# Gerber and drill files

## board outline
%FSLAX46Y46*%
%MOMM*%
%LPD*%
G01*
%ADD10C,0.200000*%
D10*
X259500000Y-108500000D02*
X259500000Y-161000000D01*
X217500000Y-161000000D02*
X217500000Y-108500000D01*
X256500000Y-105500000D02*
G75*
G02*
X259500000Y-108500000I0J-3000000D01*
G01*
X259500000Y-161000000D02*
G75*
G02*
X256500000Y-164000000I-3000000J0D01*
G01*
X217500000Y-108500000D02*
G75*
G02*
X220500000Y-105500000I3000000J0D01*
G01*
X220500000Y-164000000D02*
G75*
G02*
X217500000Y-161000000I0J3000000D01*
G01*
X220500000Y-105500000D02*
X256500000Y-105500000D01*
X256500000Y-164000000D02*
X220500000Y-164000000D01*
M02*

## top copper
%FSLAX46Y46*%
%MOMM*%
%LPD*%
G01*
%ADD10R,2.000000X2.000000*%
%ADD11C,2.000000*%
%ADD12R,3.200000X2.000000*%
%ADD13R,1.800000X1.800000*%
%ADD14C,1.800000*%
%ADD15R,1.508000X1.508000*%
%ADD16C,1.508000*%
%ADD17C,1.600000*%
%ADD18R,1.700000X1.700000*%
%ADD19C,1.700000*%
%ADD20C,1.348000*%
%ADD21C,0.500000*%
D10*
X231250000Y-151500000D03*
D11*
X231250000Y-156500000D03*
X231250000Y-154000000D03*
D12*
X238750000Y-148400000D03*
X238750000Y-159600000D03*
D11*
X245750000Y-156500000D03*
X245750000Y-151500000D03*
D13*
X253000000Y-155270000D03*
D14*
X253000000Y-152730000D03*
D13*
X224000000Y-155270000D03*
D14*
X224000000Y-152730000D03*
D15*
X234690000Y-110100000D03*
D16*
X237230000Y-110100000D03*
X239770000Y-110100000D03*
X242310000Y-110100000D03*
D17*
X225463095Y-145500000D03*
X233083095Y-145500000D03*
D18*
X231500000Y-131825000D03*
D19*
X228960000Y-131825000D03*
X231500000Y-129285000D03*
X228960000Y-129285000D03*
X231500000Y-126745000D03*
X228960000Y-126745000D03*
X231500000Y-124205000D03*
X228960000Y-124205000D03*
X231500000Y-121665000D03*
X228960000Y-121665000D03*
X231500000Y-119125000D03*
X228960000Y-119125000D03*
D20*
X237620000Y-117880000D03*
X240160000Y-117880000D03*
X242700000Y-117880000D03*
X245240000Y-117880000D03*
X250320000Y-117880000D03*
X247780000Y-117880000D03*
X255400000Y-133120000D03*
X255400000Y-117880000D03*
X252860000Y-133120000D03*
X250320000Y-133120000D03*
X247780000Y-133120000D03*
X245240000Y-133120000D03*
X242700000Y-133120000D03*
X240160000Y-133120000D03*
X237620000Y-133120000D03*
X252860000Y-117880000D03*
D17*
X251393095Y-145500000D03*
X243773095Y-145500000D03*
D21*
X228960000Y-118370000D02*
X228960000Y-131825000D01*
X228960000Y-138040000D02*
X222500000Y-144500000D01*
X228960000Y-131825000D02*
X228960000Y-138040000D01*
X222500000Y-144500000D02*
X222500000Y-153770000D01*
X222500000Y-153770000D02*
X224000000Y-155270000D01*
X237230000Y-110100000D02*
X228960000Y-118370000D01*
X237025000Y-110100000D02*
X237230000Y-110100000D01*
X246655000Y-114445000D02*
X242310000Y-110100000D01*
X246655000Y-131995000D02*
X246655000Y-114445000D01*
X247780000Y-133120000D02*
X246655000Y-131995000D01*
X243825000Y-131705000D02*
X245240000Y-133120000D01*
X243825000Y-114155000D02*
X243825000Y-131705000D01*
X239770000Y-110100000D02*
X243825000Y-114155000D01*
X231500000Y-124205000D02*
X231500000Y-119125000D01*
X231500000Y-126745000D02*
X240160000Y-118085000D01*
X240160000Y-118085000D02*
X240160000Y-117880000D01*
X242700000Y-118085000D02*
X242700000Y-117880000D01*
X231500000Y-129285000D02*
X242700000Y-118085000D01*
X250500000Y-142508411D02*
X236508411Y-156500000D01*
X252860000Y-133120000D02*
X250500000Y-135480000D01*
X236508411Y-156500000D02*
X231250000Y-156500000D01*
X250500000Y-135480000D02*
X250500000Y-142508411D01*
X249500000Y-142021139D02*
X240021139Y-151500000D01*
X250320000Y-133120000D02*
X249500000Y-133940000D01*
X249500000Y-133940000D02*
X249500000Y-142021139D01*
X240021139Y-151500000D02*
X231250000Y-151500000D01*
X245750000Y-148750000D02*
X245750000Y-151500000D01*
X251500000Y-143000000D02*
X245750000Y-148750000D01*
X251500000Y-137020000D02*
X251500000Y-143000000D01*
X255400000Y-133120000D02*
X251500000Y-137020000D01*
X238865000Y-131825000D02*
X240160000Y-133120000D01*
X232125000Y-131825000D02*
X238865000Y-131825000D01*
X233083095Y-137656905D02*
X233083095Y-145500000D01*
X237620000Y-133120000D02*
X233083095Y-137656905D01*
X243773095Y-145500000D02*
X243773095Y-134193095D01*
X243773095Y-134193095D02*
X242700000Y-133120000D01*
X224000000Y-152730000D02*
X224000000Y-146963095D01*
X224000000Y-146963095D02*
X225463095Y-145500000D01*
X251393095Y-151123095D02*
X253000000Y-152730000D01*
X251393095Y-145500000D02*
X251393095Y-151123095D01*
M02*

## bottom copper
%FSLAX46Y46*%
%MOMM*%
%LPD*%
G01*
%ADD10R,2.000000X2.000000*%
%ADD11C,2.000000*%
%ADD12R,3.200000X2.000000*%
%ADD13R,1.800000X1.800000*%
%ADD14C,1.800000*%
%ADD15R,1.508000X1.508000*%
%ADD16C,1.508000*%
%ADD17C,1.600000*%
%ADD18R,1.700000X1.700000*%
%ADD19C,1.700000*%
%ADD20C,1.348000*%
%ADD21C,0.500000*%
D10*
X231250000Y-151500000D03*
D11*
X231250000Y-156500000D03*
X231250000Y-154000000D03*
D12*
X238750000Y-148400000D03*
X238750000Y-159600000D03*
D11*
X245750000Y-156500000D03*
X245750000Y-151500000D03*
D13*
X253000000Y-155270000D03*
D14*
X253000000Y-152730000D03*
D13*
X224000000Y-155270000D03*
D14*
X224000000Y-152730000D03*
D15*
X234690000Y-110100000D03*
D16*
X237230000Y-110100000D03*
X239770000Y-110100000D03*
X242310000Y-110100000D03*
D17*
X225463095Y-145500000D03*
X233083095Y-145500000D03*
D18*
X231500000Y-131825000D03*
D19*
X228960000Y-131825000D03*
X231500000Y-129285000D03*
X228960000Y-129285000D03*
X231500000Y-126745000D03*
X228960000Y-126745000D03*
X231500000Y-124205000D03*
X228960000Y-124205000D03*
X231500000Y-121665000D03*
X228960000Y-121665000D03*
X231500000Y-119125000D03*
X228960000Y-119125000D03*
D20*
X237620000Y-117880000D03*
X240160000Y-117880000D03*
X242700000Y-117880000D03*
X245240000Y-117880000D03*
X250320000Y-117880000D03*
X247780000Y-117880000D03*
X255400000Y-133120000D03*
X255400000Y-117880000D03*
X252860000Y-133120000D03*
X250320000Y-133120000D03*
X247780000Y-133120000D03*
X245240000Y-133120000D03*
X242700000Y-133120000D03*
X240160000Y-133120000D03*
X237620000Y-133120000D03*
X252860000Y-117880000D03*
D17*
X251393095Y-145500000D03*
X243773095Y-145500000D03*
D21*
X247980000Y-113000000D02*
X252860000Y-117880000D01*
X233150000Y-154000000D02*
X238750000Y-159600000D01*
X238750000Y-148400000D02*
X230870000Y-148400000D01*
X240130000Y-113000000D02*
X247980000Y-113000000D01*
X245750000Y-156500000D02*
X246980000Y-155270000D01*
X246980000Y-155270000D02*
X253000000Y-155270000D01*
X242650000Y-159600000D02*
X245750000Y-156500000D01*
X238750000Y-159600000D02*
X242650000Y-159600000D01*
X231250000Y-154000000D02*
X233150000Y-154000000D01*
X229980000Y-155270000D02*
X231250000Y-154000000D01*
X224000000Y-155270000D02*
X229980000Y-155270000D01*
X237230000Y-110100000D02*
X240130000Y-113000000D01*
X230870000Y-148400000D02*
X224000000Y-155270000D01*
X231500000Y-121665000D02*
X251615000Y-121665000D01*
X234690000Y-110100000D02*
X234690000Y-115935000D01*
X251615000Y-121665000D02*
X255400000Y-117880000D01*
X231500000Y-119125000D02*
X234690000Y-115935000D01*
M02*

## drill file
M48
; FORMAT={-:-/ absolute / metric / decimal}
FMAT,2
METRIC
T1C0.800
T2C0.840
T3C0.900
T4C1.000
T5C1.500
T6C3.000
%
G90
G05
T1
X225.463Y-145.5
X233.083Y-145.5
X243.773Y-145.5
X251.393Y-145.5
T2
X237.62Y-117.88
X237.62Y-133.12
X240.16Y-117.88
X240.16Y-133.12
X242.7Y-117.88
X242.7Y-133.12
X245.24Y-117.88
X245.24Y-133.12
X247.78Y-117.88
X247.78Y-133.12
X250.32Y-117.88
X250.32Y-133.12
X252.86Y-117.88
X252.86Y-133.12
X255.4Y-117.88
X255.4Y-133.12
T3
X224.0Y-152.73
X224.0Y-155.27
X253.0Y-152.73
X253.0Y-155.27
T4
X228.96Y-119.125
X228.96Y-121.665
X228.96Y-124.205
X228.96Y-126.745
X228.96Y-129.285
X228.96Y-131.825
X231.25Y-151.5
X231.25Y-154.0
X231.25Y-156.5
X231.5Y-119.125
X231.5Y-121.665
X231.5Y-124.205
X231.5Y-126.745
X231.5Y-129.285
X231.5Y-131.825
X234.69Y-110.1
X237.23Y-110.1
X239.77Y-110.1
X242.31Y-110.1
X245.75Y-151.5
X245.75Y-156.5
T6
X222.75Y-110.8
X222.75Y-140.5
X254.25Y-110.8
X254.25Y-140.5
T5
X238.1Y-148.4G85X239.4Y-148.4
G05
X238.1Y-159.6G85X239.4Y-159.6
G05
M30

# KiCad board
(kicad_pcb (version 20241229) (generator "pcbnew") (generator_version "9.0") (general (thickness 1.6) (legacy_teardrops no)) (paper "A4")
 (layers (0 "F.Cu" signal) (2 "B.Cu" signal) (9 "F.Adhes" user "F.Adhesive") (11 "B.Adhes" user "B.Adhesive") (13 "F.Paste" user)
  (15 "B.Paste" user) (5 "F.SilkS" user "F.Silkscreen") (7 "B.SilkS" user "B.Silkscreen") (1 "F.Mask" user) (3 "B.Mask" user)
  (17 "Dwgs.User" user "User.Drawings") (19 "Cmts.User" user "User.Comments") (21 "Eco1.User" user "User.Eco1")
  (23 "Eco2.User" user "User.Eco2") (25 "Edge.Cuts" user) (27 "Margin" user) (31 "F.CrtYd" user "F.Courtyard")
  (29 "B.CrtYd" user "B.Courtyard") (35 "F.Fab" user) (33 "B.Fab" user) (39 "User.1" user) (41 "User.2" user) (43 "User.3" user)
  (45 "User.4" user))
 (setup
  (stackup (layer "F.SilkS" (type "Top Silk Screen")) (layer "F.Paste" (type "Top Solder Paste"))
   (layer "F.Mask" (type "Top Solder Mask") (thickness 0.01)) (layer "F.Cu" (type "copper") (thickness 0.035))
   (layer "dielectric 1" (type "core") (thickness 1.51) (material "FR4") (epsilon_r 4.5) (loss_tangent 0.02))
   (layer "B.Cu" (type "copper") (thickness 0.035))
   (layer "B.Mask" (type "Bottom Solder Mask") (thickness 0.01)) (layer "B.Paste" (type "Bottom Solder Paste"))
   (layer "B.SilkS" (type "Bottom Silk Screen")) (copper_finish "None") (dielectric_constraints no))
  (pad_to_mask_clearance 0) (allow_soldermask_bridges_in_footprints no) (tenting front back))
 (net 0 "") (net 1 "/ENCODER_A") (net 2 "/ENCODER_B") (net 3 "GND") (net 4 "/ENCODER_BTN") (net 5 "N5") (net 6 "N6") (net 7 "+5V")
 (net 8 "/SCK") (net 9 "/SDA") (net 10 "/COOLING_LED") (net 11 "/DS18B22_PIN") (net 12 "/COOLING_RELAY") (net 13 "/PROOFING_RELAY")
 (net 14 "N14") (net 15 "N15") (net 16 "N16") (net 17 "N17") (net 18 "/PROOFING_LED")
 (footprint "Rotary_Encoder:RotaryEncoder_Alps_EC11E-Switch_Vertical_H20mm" (layer "F.Cu") (at 231.25 151.5)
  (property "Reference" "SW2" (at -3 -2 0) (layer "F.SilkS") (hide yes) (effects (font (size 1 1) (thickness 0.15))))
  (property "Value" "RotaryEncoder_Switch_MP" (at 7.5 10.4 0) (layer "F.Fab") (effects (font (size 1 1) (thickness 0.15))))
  (pad "A" thru_hole rect (at 0 0) (size 2 2) (drill 1) (layers "*.Cu" "*.Mask") (remove_unused_layers no) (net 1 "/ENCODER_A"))
  (pad "B" thru_hole circle (at 0 5) (size 2 2) (drill 1) (layers "*.Cu" "*.Mask") (remove_unused_layers no) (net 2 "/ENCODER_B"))
  (pad "C" thru_hole circle (at 0 2.5) (size 2 2) (drill 1) (layers "*.Cu" "*.Mask") (remove_unused_layers no) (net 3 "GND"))
  (pad "MP" thru_hole rect (at 7.5 -3.1) (size 3.2 2) (drill oval 2.8 1.5) (layers "*.Cu" "*.Mask") (remove_unused_layers no) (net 3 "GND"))
  (pad "MP" thru_hole rect (at 7.5 8.1) (size 3.2 2) (drill oval 2.8 1.5) (layers "*.Cu" "*.Mask") (remove_unused_layers no) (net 3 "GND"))
  (pad "S1" thru_hole circle (at 14.5 5) (size 2 2) (drill 1) (layers "*.Cu" "*.Mask") (remove_unused_layers no) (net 3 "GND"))
  (pad "S2" thru_hole circle (at 14.5 0) (size 2 2) (drill 1) (layers "*.Cu" "*.Mask") (remove_unused_layers no) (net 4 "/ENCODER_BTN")))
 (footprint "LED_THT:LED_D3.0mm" (layer "F.Cu") (at 253 155.27 90)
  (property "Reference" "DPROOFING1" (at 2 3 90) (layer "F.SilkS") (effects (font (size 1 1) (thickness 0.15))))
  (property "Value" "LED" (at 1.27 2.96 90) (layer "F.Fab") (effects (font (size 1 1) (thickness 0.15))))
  (pad "1" thru_hole rect (at 0 0 90) (size 1.8 1.8) (drill 0.9) (layers "*.Cu" "*.Mask") (remove_unused_layers no) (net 3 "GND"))
  (pad "2" thru_hole circle (at 2.54 0 90) (size 1.8 1.8) (drill 0.9) (layers "*.Cu" "*.Mask") (remove_unused_layers no) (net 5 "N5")))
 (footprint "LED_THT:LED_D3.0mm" (layer "F.Cu") (at 224 155.27 90)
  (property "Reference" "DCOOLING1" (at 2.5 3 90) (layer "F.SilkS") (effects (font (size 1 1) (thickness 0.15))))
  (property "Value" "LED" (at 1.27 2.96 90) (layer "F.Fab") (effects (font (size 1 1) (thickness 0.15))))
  (pad "1" thru_hole rect (at 0 0 90) (size 1.8 1.8) (drill 0.9) (layers "*.Cu" "*.Mask") (remove_unused_layers no) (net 3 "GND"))
  (pad "2" thru_hole circle (at 2.54 0 90) (size 1.8 1.8) (drill 0.9) (layers "*.Cu" "*.Mask") (remove_unused_layers no) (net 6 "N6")))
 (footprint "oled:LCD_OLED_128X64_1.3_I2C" (layer "F.Cu") (at 238.5 125.65)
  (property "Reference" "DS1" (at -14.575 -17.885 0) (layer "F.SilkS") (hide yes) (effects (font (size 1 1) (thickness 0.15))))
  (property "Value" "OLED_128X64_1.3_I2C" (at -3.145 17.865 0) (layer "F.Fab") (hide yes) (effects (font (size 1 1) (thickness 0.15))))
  (pad "" np_thru_hole circle (at -15.75 -14.85) (size 3 3) (drill 3) (layers "*.Cu" "*.Mask"))
  (pad "" np_thru_hole circle (at -15.75 14.85) (size 3 3) (drill 3) (layers "*.Cu" "*.Mask"))
  (pad "" np_thru_hole circle (at 15.75 -14.85) (size 3 3) (drill 3) (layers "*.Cu" "*.Mask"))
  (pad "" np_thru_hole circle (at 15.75 14.85) (size 3 3) (drill 3) (layers "*.Cu" "*.Mask"))
  (pad "1" thru_hole rect (at -3.81 -15.55) (size 1.508 1.508) (drill 1) (layers "*.Cu" "*.Mask") (remove_unused_layers no) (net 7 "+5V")
   (solder_mask_margin 0.102))
  (pad "2" thru_hole circle (at -1.27 -15.55) (size 1.508 1.508) (drill 1) (layers "*.Cu" "*.Mask") (remove_unused_layers no) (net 3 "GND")
   (solder_mask_margin 0.102))
  (pad "3" thru_hole circle (at 1.27 -15.55) (size 1.508 1.508) (drill 1) (layers "*.Cu" "*.Mask") (remove_unused_layers no) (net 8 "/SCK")
   (solder_mask_margin 0.102))
  (pad "4" thru_hole circle (at 3.81 -15.55) (size 1.508 1.508) (drill 1) (layers "*.Cu" "*.Mask") (remove_unused_layers no) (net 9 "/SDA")
   (solder_mask_margin 0.102)))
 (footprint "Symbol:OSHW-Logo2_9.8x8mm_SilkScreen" (layer "B.Cu") (at 238.75 154 180)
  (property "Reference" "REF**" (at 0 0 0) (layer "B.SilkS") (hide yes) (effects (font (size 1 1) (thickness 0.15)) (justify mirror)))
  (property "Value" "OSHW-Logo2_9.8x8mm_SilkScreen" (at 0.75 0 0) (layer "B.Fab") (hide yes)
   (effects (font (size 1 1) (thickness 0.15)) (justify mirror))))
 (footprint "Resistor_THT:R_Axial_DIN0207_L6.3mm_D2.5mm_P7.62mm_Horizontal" (layer "B.Cu") (at 225.463095 145.5)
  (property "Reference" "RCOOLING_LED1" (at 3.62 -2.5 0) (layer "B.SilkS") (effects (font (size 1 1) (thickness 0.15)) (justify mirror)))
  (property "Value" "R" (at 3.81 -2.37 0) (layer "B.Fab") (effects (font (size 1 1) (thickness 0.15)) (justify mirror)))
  (pad "1" thru_hole circle (at 0 0) (size 1.6 1.6) (drill 0.8) (layers "*.Cu" "*.Mask") (remove_unused_layers no) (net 6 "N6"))
  (pad "2" thru_hole circle (at 7.62 0) (size 1.6 1.6) (drill 0.8) (layers "*.Cu" "*.Mask") (remove_unused_layers no)
   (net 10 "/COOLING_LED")))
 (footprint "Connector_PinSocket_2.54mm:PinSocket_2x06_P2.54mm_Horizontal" (layer "B.Cu") (at 231.5 131.825)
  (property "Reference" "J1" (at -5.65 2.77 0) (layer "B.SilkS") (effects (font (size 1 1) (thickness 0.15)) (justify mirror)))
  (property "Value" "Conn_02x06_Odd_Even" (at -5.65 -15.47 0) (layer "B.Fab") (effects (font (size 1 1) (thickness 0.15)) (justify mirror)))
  (pad "1" thru_hole rect (at 0 0) (size 1.7 1.7) (drill 1) (layers "*.Cu" "*.Mask") (remove_unused_layers no) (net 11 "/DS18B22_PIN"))
  (pad "2" thru_hole circle (at -2.54 0) (size 1.7 1.7) (drill 1) (layers "*.Cu" "*.Mask") (remove_unused_layers no) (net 3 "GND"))
  (pad "3" thru_hole circle (at 0 -2.54) (size 1.7 1.7) (drill 1) (layers "*.Cu" "*.Mask") (remove_unused_layers no)
   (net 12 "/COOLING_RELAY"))
  (pad "4" thru_hole circle (at -2.54 -2.54) (size 1.7 1.7) (drill 1) (layers "*.Cu" "*.Mask") (remove_unused_layers no) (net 3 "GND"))
  (pad "5" thru_hole circle (at 0 -5.08) (size 1.7 1.7) (drill 1) (layers "*.Cu" "*.Mask") (remove_unused_layers no)
   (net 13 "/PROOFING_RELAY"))
  (pad "6" thru_hole circle (at -2.54 -5.08) (size 1.7 1.7) (drill 1) (layers "*.Cu" "*.Mask") (remove_unused_layers no) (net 3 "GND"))
  (pad "7" thru_hole circle (at 0 -7.62) (size 1.7 1.7) (drill 1) (layers "*.Cu" "*.Mask") (remove_unused_layers no) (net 7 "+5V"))
  (pad "8" thru_hole circle (at -2.54 -7.62) (size 1.7 1.7) (drill 1) (layers "*.Cu" "*.Mask") (remove_unused_layers no) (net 3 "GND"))
  (pad "9" thru_hole circle (at 0 -10.16) (size 1.7 1.7) (drill 1) (layers "*.Cu" "*.Mask") (remove_unused_layers no) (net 7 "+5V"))
  (pad "10" thru_hole circle (at -2.54 -10.16) (size 1.7 1.7) (drill 1) (layers "*.Cu" "*.Mask") (remove_unused_layers no) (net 3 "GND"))
  (pad "11" thru_hole circle (at 0 -12.7) (size 1.7 1.7) (drill 1) (layers "*.Cu" "*.Mask") (remove_unused_layers no) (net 7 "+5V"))
  (pad "12" thru_hole circle (at -2.54 -12.7) (size 1.7 1.7) (drill 1) (layers "*.Cu" "*.Mask") (remove_unused_layers no) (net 3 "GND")))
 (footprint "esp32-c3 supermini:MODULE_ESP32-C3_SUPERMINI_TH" (layer "B.Cu") (at 245.5 125.5 90)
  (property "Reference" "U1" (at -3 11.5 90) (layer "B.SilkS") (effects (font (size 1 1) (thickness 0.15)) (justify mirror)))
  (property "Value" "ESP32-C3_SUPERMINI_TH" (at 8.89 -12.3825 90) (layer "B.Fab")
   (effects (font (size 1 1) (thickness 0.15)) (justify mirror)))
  (pad "0" thru_hole circle (at 7.62 -7.88 90) (size 1.348 1.348) (drill 0.84) (layers "*.Cu" "*.Mask") (remove_unused_layers no)
   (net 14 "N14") (solder_mask_margin 0.102))
  (pad "1" thru_hole circle (at 7.62 -5.34 90) (size 1.348 1.348) (drill 0.84) (layers "*.Cu" "*.Mask") (remove_unused_layers no)
   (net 13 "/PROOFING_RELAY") (solder_mask_margin 0.102))
  (pad "2" thru_hole circle (at 7.62 -2.8 90) (size 1.348 1.348) (drill 0.84) (layers "*.Cu" "*.Mask") (remove_unused_layers no)
   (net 12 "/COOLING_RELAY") (solder_mask_margin 0.102))
  (pad "3" thru_hole circle (at 7.62 -0.26 90) (size 1.348 1.348) (drill 0.84) (layers "*.Cu" "*.Mask") (remove_unused_layers no)
   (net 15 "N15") (solder_mask_margin 0.102))
  (pad "3.3" thru_hole circle (at 7.62 4.82 90) (size 1.348 1.348) (drill 0.84) (layers "*.Cu" "*.Mask") (remove_unused_layers no)
   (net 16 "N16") (solder_mask_margin 0.102))
  (pad "4" thru_hole circle (at 7.62 2.28 90) (size 1.348 1.348) (drill 0.84) (layers "*.Cu" "*.Mask") (remove_unused_layers no)
   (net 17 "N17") (solder_mask_margin 0.102))
  (pad "5" thru_hole circle (at -7.62 9.9 90) (size 1.348 1.348) (drill 0.84) (layers "*.Cu" "*.Mask") (remove_unused_layers no)
   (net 4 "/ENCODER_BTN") (solder_mask_margin 0.102))
  (pad "5V" thru_hole circle (at 7.62 9.9 90) (size 1.348 1.348) (drill 0.84) (layers "*.Cu" "*.Mask") (remove_unused_layers no)
   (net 7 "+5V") (solder_mask_margin 0.102))
  (pad "6" thru_hole circle (at -7.62 7.36 90) (size 1.348 1.348) (drill 0.84) (layers "*.Cu" "*.Mask") (remove_unused_layers no)
   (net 2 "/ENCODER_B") (solder_mask_margin 0.102))
  (pad "7" thru_hole circle (at -7.62 4.82 90) (size 1.348 1.348) (drill 0.84) (layers "*.Cu" "*.Mask") (remove_unused_layers no)
   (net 1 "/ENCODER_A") (solder_mask_margin 0.102))
  (pad "8" thru_hole circle (at -7.62 2.28 90) (size 1.348 1.348) (drill 0.84) (layers "*.Cu" "*.Mask") (remove_unused_layers no)
   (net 9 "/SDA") (solder_mask_margin 0.102))
  (pad "9" thru_hole circle (at -7.62 -0.26 90) (size 1.348 1.348) (drill 0.84) (layers "*.Cu" "*.Mask") (remove_unused_layers no)
   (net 8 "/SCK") (solder_mask_margin 0.102))
  (pad "10" thru_hole circle (at -7.62 -2.8 90) (size 1.348 1.348) (drill 0.84) (layers "*.Cu" "*.Mask") (remove_unused_layers no)
   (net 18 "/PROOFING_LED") (solder_mask_margin 0.102))
  (pad "20" thru_hole circle (at -7.62 -5.34 90) (size 1.348 1.348) (drill 0.84) (layers "*.Cu" "*.Mask") (remove_unused_layers no)
   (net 11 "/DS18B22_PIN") (solder_mask_margin 0.102))
  (pad "21" thru_hole circle (at -7.62 -7.88 90) (size 1.348 1.348) (drill 0.84) (layers "*.Cu" "*.Mask") (remove_unused_layers no)
   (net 10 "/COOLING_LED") (solder_mask_margin 0.102))
  (pad "G" thru_hole circle (at 7.62 7.36 90) (size 1.348 1.348) (drill 0.84) (layers "*.Cu" "*.Mask") (remove_unused_layers no)
   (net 3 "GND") (solder_mask_margin 0.102)))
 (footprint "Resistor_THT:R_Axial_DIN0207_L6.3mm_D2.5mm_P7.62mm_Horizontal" (layer "B.Cu") (at 251.393095 145.5 180)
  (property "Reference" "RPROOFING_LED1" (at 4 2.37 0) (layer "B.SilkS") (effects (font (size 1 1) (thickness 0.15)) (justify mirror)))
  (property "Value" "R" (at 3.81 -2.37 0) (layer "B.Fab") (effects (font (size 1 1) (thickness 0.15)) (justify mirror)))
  (pad "1" thru_hole circle (at 0 0 180) (size 1.6 1.6) (drill 0.8) (layers "*.Cu" "*.Mask") (remove_unused_layers no) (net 5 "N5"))
  (pad "2" thru_hole circle (at 7.62 0 180) (size 1.6 1.6) (drill 0.8) (layers "*.Cu" "*.Mask") (remove_unused_layers no)
   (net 18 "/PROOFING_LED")))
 (gr_line (start 259.5 108.5) (end 259.5 161) (stroke (width 0.2) (type default)) (layer "Edge.Cuts"))
 (gr_line (start 217.5 161) (end 217.5 108.5) (stroke (width 0.2) (type default)) (layer "Edge.Cuts"))
 (gr_arc (start 256.5 105.5) (mid 258.62132 106.37868) (end 259.5 108.5) (stroke (width 0.2) (type default)) (layer "Edge.Cuts"))
 (gr_arc (start 259.5 161) (mid 258.62132 163.12132) (end 256.5 164) (stroke (width 0.2) (type default)) (layer "Edge.Cuts"))
 (gr_arc (start 217.5 108.5) (mid 218.37868 106.37868) (end 220.5 105.5) (stroke (width 0.2) (type default)) (layer "Edge.Cuts"))
 (gr_arc (start 220.5 164) (mid 218.37868 163.12132) (end 217.5 161) (stroke (width 0.2) (type default)) (layer "Edge.Cuts"))
 (gr_line (start 220.5 105.5) (end 256.5 105.5) (stroke (width 0.2) (type default)) (layer "Edge.Cuts"))
 (gr_line (start 256.5 164) (end 220.5 164) (stroke (width 0.2) (type default)) (layer "Edge.Cuts"))
 (segment (start 228.96 118.37) (end 228.96 131.825) (width 0.5) (layer "F.Cu") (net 3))
 (segment (start 228.96 138.04) (end 222.5 144.5) (width 0.5) (layer "F.Cu") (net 3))
 (segment (start 228.96 131.825) (end 228.96 138.04) (width 0.5) (layer "F.Cu") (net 3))
 (segment (start 222.5 144.5) (end 222.5 153.77) (width 0.5) (layer "F.Cu") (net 3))
 (segment (start 222.5 153.77) (end 224 155.27) (width 0.5) (layer "F.Cu") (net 3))
 (segment (start 237.23 110.1) (end 228.96 118.37) (width 0.5) (layer "F.Cu") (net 3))
 (segment (start 237.025 110.1) (end 237.23 110.1) (width 0.5) (layer "F.Cu") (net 3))
 (segment (start 247.98 113) (end 252.86 117.88) (width 0.5) (layer "B.Cu") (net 3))
 (segment (start 233.15 154) (end 238.75 159.6) (width 0.5) (layer "B.Cu") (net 3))
 (segment (start 238.75 148.4) (end 230.87 148.4) (width 0.5) (layer "B.Cu") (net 3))
 (segment (start 240.13 113) (end 247.98 113) (width 0.5) (layer "B.Cu") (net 3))
 (segment (start 245.75 156.5) (end 246.98 155.27) (width 0.5) (layer "B.Cu") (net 3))
 (segment (start 246.98 155.27) (end 253 155.27) (width 0.5) (layer "B.Cu") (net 3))
 (segment (start 242.65 159.6) (end 245.75 156.5) (width 0.5) (layer "B.Cu") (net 3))
 (segment (start 238.75 159.6) (end 242.65 159.6) (width 0.5) (layer "B.Cu") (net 3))
 (segment (start 231.25 154) (end 233.15 154) (width 0.5) (layer "B.Cu") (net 3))
 (segment (start 229.98 155.27) (end 231.25 154) (width 0.5) (layer "B.Cu") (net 3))
 (segment (start 224 155.27) (end 229.98 155.27) (width 0.5) (layer "B.Cu") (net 3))
 (segment (start 237.23 110.1) (end 240.13 113) (width 0.5) (layer "B.Cu") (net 3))
 (segment (start 230.87 148.4) (end 224 155.27) (width 0.5) (layer "B.Cu") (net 3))
 (segment (start 246.655 114.445) (end 242.31 110.1) (width 0.5) (layer "F.Cu") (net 9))
 (segment (start 246.655 131.995) (end 246.655 114.445) (width 0.5) (layer "F.Cu") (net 9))
 (segment (start 247.78 133.12) (end 246.655 131.995) (width 0.5) (layer "F.Cu") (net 9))
 (segment (start 243.825 131.705) (end 245.24 133.12) (width 0.5) (layer "F.Cu") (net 8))
 (segment (start 243.825 114.155) (end 243.825 131.705) (width 0.5) (layer "F.Cu") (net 8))
 (segment (start 239.77 110.1) (end 243.825 114.155) (width 0.5) (layer "F.Cu") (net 8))
 (segment (start 231.5 124.205) (end 231.5 119.125) (width 0.5) (layer "F.Cu") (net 7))
 (segment (start 231.5 121.665) (end 251.615 121.665) (width 0.5) (layer "B.Cu") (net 7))
 (segment (start 234.69 110.1) (end 234.69 115.935) (width 0.5) (layer "B.Cu") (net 7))
 (segment (start 251.615 121.665) (end 255.4 117.88) (width 0.5) (layer "B.Cu") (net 7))
 (segment (start 231.5 119.125) (end 234.69 115.935) (width 0.5) (layer "B.Cu") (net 7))
 (segment (start 231.5 126.745) (end 240.16 118.085) (width 0.5) (layer "F.Cu") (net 13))
 (segment (start 240.16 118.085) (end 240.16 117.88) (width 0.5) (layer "F.Cu") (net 13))
 (segment (start 242.7 118.085) (end 242.7 117.88) (width 0.5) (layer "F.Cu") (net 12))
 (segment (start 231.5 129.285) (end 242.7 118.085) (width 0.5) (layer "F.Cu") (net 12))
 (segment (start 250.5 142.508411) (end 236.508411 156.5) (width 0.5) (layer "F.Cu") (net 2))
 (segment (start 252.86 133.12) (end 250.5 135.48) (width 0.5) (layer "F.Cu") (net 2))
 (segment (start 236.508411 156.5) (end 231.25 156.5) (width 0.5) (layer "F.Cu") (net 2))
 (segment (start 250.5 135.48) (end 250.5 142.508411) (width 0.5) (layer "F.Cu") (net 2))
 (segment (start 249.5 142.021139) (end 240.021139 151.5) (width 0.5) (layer "F.Cu") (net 1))
 (segment (start 250.32 133.12) (end 249.5 133.94) (width 0.5) (layer "F.Cu") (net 1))
 (segment (start 249.5 133.94) (end 249.5 142.021139) (width 0.5) (layer "F.Cu") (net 1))
 (segment (start 240.021139 151.5) (end 231.25 151.5) (width 0.5) (layer "F.Cu") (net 1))
 (segment (start 245.75 148.75) (end 245.75 151.5) (width 0.5) (layer "F.Cu") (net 4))
 (segment (start 251.5 143) (end 245.75 148.75) (width 0.5) (layer "F.Cu") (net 4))
 (segment (start 251.5 137.02) (end 251.5 143) (width 0.5) (layer "F.Cu") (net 4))
 (segment (start 255.4 133.12) (end 251.5 137.02) (width 0.5) (layer "F.Cu") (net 4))
 (segment (start 238.865 131.825) (end 240.16 133.12) (width 0.5) (layer "F.Cu") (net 11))
 (segment (start 232.125 131.825) (end 238.865 131.825) (width 0.5) (layer "F.Cu") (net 11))
 (segment (start 233.083095 137.656905) (end 233.083095 145.5) (width 0.5) (layer "F.Cu") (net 10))
 (segment (start 237.62 133.12) (end 233.083095 137.656905) (width 0.5) (layer "F.Cu") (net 10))
 (segment (start 243.773095 145.5) (end 243.773095 134.193095) (width 0.5) (layer "F.Cu") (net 18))
 (segment (start 243.773095 134.193095) (end 242.7 133.12) (width 0.5) (layer "F.Cu") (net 18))
 (segment (start 224 152.73) (end 224 146.963095) (width 0.5) (layer "F.Cu") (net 6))
 (segment (start 224 146.963095) (end 225.463095 145.5) (width 0.5) (layer "F.Cu") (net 6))
 (segment (start 251.393095 151.123095) (end 253 152.73) (width 0.5) (layer "F.Cu") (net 5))
 (segment (start 251.393095 145.5) (end 251.393095 151.123095) (width 0.5) (layer "F.Cu") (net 5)))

